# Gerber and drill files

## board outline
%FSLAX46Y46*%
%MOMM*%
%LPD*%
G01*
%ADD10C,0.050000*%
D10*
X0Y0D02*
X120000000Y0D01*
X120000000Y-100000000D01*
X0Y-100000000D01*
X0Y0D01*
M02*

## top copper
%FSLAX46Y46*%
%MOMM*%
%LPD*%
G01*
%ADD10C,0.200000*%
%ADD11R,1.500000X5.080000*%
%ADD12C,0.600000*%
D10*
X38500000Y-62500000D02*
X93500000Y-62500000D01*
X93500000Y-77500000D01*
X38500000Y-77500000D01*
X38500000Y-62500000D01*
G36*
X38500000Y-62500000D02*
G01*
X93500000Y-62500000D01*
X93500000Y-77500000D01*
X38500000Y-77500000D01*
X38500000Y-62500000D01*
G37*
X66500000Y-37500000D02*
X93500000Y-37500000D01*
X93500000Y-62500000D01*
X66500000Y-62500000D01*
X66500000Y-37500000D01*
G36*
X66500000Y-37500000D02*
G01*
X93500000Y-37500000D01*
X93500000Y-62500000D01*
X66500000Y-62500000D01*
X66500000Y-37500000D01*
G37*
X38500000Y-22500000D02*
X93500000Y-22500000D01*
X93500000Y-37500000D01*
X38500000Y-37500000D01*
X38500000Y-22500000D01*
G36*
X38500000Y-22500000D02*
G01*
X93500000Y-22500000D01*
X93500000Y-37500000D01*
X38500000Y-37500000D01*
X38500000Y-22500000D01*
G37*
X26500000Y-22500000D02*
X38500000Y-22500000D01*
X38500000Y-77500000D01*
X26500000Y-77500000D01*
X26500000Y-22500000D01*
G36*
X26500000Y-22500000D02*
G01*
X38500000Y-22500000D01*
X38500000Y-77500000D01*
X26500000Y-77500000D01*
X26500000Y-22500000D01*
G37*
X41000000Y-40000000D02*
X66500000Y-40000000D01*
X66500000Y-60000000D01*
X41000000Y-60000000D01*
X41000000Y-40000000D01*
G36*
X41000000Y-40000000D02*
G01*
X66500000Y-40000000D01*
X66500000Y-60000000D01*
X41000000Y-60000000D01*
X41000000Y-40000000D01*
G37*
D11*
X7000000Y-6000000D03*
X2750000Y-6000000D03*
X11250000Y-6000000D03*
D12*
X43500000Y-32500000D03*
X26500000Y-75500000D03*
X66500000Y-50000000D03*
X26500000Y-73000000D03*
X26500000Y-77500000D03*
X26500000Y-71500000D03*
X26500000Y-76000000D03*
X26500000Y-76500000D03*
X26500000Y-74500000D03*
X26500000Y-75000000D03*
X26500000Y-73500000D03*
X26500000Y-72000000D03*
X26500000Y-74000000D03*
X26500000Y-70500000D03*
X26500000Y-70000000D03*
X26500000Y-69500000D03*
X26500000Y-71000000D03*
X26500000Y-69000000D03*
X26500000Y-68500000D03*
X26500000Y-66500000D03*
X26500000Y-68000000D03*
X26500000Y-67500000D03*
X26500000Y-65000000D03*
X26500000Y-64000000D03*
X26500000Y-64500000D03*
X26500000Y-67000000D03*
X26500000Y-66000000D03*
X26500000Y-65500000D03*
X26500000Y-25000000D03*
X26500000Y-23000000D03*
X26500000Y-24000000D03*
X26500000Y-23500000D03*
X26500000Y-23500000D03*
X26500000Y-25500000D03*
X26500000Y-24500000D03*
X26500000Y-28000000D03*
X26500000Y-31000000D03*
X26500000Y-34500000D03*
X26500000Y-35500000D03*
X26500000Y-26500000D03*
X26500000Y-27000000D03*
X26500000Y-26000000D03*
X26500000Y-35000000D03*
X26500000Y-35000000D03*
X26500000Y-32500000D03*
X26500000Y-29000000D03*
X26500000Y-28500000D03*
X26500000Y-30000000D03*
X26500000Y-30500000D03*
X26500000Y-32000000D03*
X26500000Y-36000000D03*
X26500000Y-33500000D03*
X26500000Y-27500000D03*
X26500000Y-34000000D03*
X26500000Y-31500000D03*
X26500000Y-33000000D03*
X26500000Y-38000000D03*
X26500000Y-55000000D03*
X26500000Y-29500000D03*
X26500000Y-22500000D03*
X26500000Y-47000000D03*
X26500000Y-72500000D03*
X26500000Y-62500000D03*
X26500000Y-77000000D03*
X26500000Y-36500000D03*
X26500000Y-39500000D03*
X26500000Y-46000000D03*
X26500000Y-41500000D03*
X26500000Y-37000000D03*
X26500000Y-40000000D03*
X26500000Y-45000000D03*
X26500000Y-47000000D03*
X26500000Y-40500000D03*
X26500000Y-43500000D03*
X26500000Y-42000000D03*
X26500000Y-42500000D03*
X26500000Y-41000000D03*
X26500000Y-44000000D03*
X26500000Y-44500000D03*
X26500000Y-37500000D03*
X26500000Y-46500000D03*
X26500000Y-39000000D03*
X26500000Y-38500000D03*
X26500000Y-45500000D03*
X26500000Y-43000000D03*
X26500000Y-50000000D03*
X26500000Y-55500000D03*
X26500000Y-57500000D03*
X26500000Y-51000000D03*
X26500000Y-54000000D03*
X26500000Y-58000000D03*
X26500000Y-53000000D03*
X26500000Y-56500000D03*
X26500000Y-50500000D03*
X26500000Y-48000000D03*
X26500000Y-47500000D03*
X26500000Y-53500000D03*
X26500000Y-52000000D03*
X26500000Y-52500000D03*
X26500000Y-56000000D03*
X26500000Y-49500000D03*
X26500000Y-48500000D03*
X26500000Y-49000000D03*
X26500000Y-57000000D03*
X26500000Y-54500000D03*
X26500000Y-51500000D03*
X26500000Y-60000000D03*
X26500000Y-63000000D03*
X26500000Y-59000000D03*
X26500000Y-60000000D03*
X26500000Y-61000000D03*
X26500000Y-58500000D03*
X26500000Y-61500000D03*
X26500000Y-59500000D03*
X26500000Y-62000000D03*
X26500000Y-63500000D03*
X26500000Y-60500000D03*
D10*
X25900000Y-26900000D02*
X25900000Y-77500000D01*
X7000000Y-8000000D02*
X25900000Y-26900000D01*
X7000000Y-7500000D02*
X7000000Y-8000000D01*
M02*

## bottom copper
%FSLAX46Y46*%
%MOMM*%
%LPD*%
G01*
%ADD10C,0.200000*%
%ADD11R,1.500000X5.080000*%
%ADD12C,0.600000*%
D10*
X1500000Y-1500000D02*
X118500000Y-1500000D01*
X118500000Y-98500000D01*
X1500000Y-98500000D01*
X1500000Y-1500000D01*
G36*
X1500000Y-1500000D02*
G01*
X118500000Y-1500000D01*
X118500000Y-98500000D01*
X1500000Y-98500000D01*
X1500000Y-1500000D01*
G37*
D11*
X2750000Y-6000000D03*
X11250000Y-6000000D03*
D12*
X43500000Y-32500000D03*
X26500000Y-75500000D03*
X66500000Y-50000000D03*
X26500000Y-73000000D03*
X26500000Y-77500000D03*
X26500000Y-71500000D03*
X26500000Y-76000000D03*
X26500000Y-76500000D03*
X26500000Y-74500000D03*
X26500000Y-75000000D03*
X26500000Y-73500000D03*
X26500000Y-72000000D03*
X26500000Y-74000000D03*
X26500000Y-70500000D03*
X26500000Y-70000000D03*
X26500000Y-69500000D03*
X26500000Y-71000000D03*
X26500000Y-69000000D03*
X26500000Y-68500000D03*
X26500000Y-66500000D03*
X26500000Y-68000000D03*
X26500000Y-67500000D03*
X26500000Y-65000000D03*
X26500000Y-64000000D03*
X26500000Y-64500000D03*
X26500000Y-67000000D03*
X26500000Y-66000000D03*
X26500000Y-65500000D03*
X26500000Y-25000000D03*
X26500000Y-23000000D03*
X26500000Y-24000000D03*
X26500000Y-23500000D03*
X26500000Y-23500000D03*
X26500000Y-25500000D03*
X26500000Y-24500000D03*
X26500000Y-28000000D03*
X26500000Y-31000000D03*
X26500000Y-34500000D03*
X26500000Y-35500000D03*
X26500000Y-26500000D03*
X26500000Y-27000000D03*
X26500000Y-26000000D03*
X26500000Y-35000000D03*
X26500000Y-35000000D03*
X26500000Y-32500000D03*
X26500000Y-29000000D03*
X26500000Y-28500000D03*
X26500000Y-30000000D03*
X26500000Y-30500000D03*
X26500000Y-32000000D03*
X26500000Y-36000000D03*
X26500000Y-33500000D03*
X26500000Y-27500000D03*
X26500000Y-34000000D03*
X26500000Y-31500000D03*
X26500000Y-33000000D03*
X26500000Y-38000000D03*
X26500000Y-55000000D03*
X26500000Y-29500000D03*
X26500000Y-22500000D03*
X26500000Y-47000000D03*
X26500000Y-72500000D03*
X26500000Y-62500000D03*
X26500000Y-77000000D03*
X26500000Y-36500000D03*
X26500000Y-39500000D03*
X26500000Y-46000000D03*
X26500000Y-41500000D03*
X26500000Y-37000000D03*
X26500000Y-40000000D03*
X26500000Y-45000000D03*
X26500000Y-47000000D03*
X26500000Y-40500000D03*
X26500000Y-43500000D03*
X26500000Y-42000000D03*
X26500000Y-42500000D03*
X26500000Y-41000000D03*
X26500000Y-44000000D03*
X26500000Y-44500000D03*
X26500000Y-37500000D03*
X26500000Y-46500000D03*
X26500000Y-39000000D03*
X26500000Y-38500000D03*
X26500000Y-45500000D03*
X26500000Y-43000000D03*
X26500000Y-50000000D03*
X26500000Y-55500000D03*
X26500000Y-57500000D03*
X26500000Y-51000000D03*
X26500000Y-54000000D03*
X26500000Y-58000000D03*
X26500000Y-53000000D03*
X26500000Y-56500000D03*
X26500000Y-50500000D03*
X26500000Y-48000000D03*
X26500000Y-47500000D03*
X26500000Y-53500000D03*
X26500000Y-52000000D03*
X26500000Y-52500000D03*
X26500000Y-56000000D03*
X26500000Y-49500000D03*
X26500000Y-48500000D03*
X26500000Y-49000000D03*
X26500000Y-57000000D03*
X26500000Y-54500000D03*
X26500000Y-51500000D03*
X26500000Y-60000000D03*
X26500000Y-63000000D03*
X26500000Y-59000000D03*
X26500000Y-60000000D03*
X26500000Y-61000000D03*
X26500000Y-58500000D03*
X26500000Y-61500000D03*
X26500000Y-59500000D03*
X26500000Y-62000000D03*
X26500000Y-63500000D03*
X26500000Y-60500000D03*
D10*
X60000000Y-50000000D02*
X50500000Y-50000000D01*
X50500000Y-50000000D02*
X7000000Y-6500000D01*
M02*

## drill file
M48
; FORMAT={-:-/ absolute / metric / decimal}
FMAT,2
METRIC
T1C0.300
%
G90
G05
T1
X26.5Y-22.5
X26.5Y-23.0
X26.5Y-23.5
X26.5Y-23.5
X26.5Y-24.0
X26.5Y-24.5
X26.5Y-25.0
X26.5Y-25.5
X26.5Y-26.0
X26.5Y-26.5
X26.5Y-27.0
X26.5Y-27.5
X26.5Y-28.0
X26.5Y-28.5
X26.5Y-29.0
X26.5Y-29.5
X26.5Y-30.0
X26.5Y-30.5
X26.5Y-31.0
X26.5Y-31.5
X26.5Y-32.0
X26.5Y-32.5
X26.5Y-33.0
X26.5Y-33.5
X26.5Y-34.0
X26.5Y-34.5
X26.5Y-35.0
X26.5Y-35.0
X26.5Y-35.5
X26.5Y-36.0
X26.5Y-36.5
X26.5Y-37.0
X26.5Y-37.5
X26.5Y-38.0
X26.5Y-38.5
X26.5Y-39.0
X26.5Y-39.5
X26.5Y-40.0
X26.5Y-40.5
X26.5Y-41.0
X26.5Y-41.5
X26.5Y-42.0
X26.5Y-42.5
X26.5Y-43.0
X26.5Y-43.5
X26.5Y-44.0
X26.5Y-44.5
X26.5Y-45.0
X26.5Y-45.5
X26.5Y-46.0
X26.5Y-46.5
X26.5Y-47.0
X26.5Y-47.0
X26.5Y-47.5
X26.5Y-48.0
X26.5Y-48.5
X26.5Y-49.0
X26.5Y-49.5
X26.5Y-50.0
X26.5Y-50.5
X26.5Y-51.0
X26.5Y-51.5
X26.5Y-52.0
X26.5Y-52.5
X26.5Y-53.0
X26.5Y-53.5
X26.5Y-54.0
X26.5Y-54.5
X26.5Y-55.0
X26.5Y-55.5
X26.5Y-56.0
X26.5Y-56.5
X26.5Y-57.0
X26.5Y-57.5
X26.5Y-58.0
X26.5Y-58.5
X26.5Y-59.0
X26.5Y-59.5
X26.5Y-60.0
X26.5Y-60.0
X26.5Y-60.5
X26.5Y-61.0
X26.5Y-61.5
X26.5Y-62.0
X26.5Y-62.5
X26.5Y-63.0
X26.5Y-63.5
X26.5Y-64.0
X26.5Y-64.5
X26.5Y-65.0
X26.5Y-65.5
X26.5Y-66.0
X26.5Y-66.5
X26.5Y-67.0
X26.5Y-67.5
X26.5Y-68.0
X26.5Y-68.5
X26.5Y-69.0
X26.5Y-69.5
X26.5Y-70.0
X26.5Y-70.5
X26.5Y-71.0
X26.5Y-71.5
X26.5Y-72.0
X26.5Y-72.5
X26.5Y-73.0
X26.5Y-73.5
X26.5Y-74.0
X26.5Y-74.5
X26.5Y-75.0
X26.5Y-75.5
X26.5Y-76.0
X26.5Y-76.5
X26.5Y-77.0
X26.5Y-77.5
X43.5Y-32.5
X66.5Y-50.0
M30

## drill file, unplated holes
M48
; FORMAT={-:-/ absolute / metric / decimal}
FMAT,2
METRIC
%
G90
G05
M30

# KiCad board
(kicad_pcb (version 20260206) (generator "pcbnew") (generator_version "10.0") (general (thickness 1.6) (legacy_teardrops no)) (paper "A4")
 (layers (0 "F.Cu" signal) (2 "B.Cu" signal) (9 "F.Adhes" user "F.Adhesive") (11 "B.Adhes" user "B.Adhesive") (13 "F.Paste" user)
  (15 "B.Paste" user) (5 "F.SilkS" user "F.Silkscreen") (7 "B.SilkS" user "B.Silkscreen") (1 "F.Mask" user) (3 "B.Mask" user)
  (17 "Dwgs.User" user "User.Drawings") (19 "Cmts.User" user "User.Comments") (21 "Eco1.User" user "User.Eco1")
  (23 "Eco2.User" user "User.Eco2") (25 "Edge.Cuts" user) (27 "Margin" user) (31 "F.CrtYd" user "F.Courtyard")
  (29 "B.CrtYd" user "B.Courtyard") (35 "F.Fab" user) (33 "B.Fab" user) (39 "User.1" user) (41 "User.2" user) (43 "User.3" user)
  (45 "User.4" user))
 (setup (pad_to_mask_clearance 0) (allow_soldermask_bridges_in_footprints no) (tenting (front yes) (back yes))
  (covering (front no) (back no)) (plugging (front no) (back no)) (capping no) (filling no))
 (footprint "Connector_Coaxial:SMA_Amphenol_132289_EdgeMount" (layer "F.Cu") (at 7 6 90)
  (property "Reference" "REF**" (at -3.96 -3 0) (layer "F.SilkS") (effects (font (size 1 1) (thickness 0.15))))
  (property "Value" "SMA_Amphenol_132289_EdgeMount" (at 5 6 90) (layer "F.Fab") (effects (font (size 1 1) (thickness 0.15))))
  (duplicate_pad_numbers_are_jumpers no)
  (pad "1" smd rect (at 0 0 180) (size 1.5 5.08) (layers "F.Cu" "F.Mask" "F.Paste") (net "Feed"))
  (pad "2" smd rect (at 0 -4.25 180) (size 1.5 5.08) (layers "F.Cu" "F.Mask" "F.Paste"))
  (pad "2" smd rect (at 0 -4.25 180) (size 1.5 5.08) (layers "B.Cu" "B.Mask" "B.Paste") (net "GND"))
  (pad "2" smd rect (at 0 4.25 180) (size 1.5 5.08) (layers "F.Cu" "F.Mask" "F.Paste"))
  (pad "2" smd rect (at 0 4.25 180) (size 1.5 5.08) (layers "B.Cu" "B.Mask" "B.Paste") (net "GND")))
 (gr_rect (start 26.5 22.5) (end 38.5 77.5) (stroke (width 0.2) (type default)) (fill yes) (layer "F.Cu") (net "GND"))
 (gr_rect (start 38.5 22.5) (end 93.5 37.5) (stroke (width 0.2) (type default)) (fill yes) (layer "F.Cu") (net "GND"))
 (gr_rect (start 38.5 62.5) (end 93.5 77.5) (stroke (width 0.2) (type default)) (fill yes) (layer "F.Cu") (net "GND"))
 (gr_rect (start 41 40) (end 66.5 60) (stroke (width 0.2) (type default)) (fill yes) (layer "F.Cu") (net "GND"))
 (gr_rect (start 66.5 37.5) (end 93.5 62.5) (stroke (width 0.2) (type default)) (fill yes) (layer "F.Cu") (net "GND"))
 (gr_rect (start 1.5 1.5) (end 118.5 98.5) (stroke (width 0.2) (type solid)) (fill yes) (layer "B.Cu") (net "GND"))
 (gr_rect (start 0 0) (end 120 100) (stroke (width 0.05) (type default)) (fill no) (layer "Edge.Cuts"))
 (segment (start 7 8) (end 25.9 26.9) (width 0.2) (layer "F.Cu") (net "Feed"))
 (segment (start 7 7.5) (end 7 8) (width 0.2) (layer "F.Cu") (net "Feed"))
 (segment (start 25.9 26.9) (end 25.9 77.5) (width 0.2) (layer "F.Cu") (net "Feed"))
 (via (at 26.5 41.5) (size 0.6) (drill 0.3) (layers "F.Cu" "B.Cu") (free yes) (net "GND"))
 (via (at 26.5 47.5) (size 0.6) (drill 0.3) (layers "F.Cu" "B.Cu") (free yes) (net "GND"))
 (via (at 26.5 51.5) (size 0.6) (drill 0.3) (layers "F.Cu" "B.Cu") (free yes) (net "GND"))
 (via (at 26.5 53.5) (size 0.6) (drill 0.3) (layers "F.Cu" "B.Cu") (free yes) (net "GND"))
 (via (at 26.5 25) (size 0.6) (drill 0.3) (layers "F.Cu" "B.Cu") (free yes) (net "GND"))
 (via (at 26.5 30) (size 0.6) (drill 0.3) (layers "F.Cu" "B.Cu") (free yes) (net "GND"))
 (via (at 26.5 55.5) (size 0.6) (drill 0.3) (layers "F.Cu" "B.Cu") (free yes) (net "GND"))
 (via (at 26.5 29) (size 0.6) (drill 0.3) (layers "F.Cu" "B.Cu") (free yes) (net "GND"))
 (via (at 26.5 35) (size 0.6) (drill 0.3) (layers "F.Cu" "B.Cu") (free yes) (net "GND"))
 (via (at 26.5 55) (size 0.6) (drill 0.3) (layers "F.Cu" "B.Cu") (free yes) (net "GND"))
 (via (at 26.5 34.5) (size 0.6) (drill 0.3) (layers "F.Cu" "B.Cu") (free yes) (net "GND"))
 (via (at 26.5 24) (size 0.6) (drill 0.3) (layers "F.Cu" "B.Cu") (free yes) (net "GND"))
 (via (at 26.5 71.5) (size 0.6) (drill 0.3) (layers "F.Cu" "B.Cu") (free yes) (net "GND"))
 (via (at 26.5 68) (size 0.6) (drill 0.3) (layers "F.Cu" "B.Cu") (free yes) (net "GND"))
 (via (at 26.5 64.5) (size 0.6) (drill 0.3) (layers "F.Cu" "B.Cu") (free yes) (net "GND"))
 (via (at 26.5 26) (size 0.6) (drill 0.3) (layers "F.Cu" "B.Cu") (free yes) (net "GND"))
 (via (at 26.5 46.5) (size 0.6) (drill 0.3) (layers "F.Cu" "B.Cu") (free yes) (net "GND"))
 (via (at 26.5 53) (size 0.6) (drill 0.3) (layers "F.Cu" "B.Cu") (free yes) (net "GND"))
 (via (at 26.5 54) (size 0.6) (drill 0.3) (layers "F.Cu" "B.Cu") (free yes) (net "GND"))
 (via (at 26.5 62) (size 0.6) (drill 0.3) (layers "F.Cu" "B.Cu") (free yes) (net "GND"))
 (via (at 26.5 32) (size 0.6) (drill 0.3) (layers "F.Cu" "B.Cu") (free yes) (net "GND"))
 (via (at 26.5 50) (size 0.6) (drill 0.3) (layers "F.Cu" "B.Cu") (free yes) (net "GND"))
 (via (at 26.5 47) (size 0.6) (drill 0.3) (layers "F.Cu" "B.Cu") (free yes) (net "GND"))
 (via (at 26.5 29.5) (size 0.6) (drill 0.3) (layers "F.Cu" "B.Cu") (free yes) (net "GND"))
 (via (at 26.5 45.5) (size 0.6) (drill 0.3) (layers "F.Cu" "B.Cu") (free yes) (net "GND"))
 (via (at 26.5 52.5) (size 0.6) (drill 0.3) (layers "F.Cu" "B.Cu") (free yes) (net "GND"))
 (via (at 26.5 68.5) (size 0.6) (drill 0.3) (layers "F.Cu" "B.Cu") (free yes) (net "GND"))
 (via (at 26.5 57) (size 0.6) (drill 0.3) (layers "F.Cu" "B.Cu") (free yes) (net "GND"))
 (via (at 26.5 33) (size 0.6) (drill 0.3) (layers "F.Cu" "B.Cu") (free yes) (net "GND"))
 (via (at 26.5 36) (size 0.6) (drill 0.3) (layers "F.Cu" "B.Cu") (free yes) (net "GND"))
 (via (at 26.5 30.5) (size 0.6) (drill 0.3) (layers "F.Cu" "B.Cu") (free yes) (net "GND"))
 (via (at 26.5 66) (size 0.6) (drill 0.3) (layers "F.Cu" "B.Cu") (free yes) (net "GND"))
 (via (at 26.5 67) (size 0.6) (drill 0.3) (layers "F.Cu" "B.Cu") (free yes) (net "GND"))
 (via (at 26.5 63.5) (size 0.6) (drill 0.3) (layers "F.Cu" "B.Cu") (free yes) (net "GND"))
 (via (at 26.5 66.5) (size 0.6) (drill 0.3) (layers "F.Cu" "B.Cu") (free yes) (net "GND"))
 (via (at 26.5 56.5) (size 0.6) (drill 0.3) (layers "F.Cu" "B.Cu") (free yes) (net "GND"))
 (via (at 26.5 61.5) (size 0.6) (drill 0.3) (layers "F.Cu" "B.Cu") (free yes) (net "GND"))
 (via (at 26.5 43.5) (size 0.6) (drill 0.3) (layers "F.Cu" "B.Cu") (free yes) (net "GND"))
 (via (at 26.5 65) (size 0.6) (drill 0.3) (layers "F.Cu" "B.Cu") (free yes) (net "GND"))
 (via (at 26.5 32.5) (size 0.6) (drill 0.3) (layers "F.Cu" "B.Cu") (free yes) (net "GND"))
 (via (at 26.5 60.5) (size 0.6) (drill 0.3) (layers "F.Cu" "B.Cu") (free yes) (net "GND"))
 (via (at 26.5 26.5) (size 0.6) (drill 0.3) (layers "F.Cu" "B.Cu") (free yes) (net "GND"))
 (via (at 26.5 77.5) (size 0.6) (drill 0.3) (layers "F.Cu" "B.Cu") (free yes) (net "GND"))
 (via (at 26.5 72.5) (size 0.6) (drill 0.3) (layers "F.Cu" "B.Cu") (free yes) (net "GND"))
 (via (at 26.5 75.5) (size 0.6) (drill 0.3) (layers "F.Cu" "B.Cu") (free yes) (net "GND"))
 (via (at 26.5 56) (size 0.6) (drill 0.3) (layers "F.Cu" "B.Cu") (free yes) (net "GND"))
 (via (at 26.5 49.5) (size 0.6) (drill 0.3) (layers "F.Cu" "B.Cu") (free yes) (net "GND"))
 (via (at 26.5 70.5) (size 0.6) (drill 0.3) (layers "F.Cu" "B.Cu") (free yes) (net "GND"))
 (via (at 26.5 49) (size 0.6) (drill 0.3) (layers "F.Cu" "B.Cu") (free yes) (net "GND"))
 (via (at 26.5 23.5) (size 0.6) (drill 0.3) (layers "F.Cu" "B.Cu") (free yes) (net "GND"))
 (via (at 26.5 67.5) (size 0.6) (drill 0.3) (layers "F.Cu" "B.Cu") (free yes) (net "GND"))
 (via (at 26.5 44) (size 0.6) (drill 0.3) (layers "F.Cu" "B.Cu") (free yes) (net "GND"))
 (via (at 26.5 60) (size 0.6) (drill 0.3) (layers "F.Cu" "B.Cu") (free yes) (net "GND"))
 (via (at 26.5 27) (size 0.6) (drill 0.3) (layers "F.Cu" "B.Cu") (free yes) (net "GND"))
 (via (at 26.5 69.5) (size 0.6) (drill 0.3) (layers "F.Cu" "B.Cu") (free yes) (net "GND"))
 (via (at 26.5 71) (size 0.6) (drill 0.3) (layers "F.Cu" "B.Cu") (free yes) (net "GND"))
 (via (at 26.5 73) (size 0.6) (drill 0.3) (layers "F.Cu" "B.Cu") (free yes) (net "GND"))
 (via (at 26.5 48.5) (size 0.6) (drill 0.3) (layers "F.Cu" "B.Cu") (free yes) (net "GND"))
 (via (at 26.5 31.5) (size 0.6) (drill 0.3) (layers "F.Cu" "B.Cu") (free yes) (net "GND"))
 (via (at 26.5 52) (size 0.6) (drill 0.3) (layers "F.Cu" "B.Cu") (free yes) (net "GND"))
 (via (at 26.5 38) (size 0.6) (drill 0.3) (layers "F.Cu" "B.Cu") (free yes) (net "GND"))
 (via (at 26.5 34) (size 0.6) (drill 0.3) (layers "F.Cu" "B.Cu") (free yes) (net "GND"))
 (via (at 26.5 27.5) (size 0.6) (drill 0.3) (layers "F.Cu" "B.Cu") (free yes) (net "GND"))
 (via (at 26.5 38.5) (size 0.6) (drill 0.3) (layers "F.Cu" "B.Cu") (free yes) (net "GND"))
 (via (at 26.5 58) (size 0.6) (drill 0.3) (layers "F.Cu" "B.Cu") (free yes) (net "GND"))
 (via (at 26.5 63) (size 0.6) (drill 0.3) (layers "F.Cu" "B.Cu") (free yes) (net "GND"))
 (via (at 26.5 64) (size 0.6) (drill 0.3) (layers "F.Cu" "B.Cu") (free yes) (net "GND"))
 (via (at 66.5 50) (size 0.6) (drill 0.3) (layers "F.Cu" "B.Cu") (free yes) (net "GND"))
 (via (at 26.5 40) (size 0.6) (drill 0.3) (layers "F.Cu" "B.Cu") (free yes) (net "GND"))
 (via (at 26.5 62.5) (size 0.6) (drill 0.3) (layers "F.Cu" "B.Cu") (free yes) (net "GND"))
 (via (at 26.5 65.5) (size 0.6) (drill 0.3) (layers "F.Cu" "B.Cu") (free yes) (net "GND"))
 (via (at 26.5 69) (size 0.6) (drill 0.3) (layers "F.Cu" "B.Cu") (free yes) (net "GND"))
 (via (at 26.5 73.5) (size 0.6) (drill 0.3) (layers "F.Cu" "B.Cu") (free yes) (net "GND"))
 (via (at 26.5 22.5) (size 0.6) (drill 0.3) (layers "F.Cu" "B.Cu") (free yes) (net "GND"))
 (via (at 26.5 61) (size 0.6) (drill 0.3) (layers "F.Cu" "B.Cu") (free yes) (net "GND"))
 (via (at 26.5 59) (size 0.6) (drill 0.3) (layers "F.Cu" "B.Cu") (free yes) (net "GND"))
 (via (at 26.5 70) (size 0.6) (drill 0.3) (layers "F.Cu" "B.Cu") (free yes) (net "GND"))
 (via (at 26.5 42.5) (size 0.6) (drill 0.3) (layers "F.Cu" "B.Cu") (free yes) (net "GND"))
 (via (at 26.5 47) (size 0.6) (drill 0.3) (layers "F.Cu" "B.Cu") (free yes) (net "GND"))
 (via (at 26.5 43) (size 0.6) (drill 0.3) (layers "F.Cu" "B.Cu") (free yes) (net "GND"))
 (via (at 26.5 28.5) (size 0.6) (drill 0.3) (layers "F.Cu" "B.Cu") (free yes) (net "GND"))
 (via (at 26.5 37.5) (size 0.6) (drill 0.3) (layers "F.Cu" "B.Cu") (free yes) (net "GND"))
 (via (at 26.5 45) (size 0.6) (drill 0.3) (layers "F.Cu" "B.Cu") (free yes) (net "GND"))
 (via (at 26.5 60) (size 0.6) (drill 0.3) (layers "F.Cu" "B.Cu") (free yes) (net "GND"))
 (via (at 26.5 58.5) (size 0.6) (drill 0.3) (layers "F.Cu" "B.Cu") (free yes) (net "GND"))
 (via (at 43.5 32.5) (size 0.6) (drill 0.3) (layers "F.Cu" "B.Cu") (free yes) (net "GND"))
 (via (at 26.5 40.5) (size 0.6) (drill 0.3) (layers "F.Cu" "B.Cu") (free yes) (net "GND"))
 (via (at 26.5 23) (size 0.6) (drill 0.3) (layers "F.Cu" "B.Cu") (free yes) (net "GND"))
 (via (at 26.5 59.5) (size 0.6) (drill 0.3) (layers "F.Cu" "B.Cu") (free yes) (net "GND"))
 (via (at 26.5 72) (size 0.6) (drill 0.3) (layers "F.Cu" "B.Cu") (free yes) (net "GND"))
 (via (at 26.5 76) (size 0.6) (drill 0.3) (layers "F.Cu" "B.Cu") (free yes) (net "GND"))
 (via (at 26.5 74.5) (size 0.6) (drill 0.3) (layers "F.Cu" "B.Cu") (free yes) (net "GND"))
 (via (at 26.5 35.5) (size 0.6) (drill 0.3) (layers "F.Cu" "B.Cu") (free yes) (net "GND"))
 (via (at 26.5 39.5) (size 0.6) (drill 0.3) (layers "F.Cu" "B.Cu") (free yes) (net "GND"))
 (via (at 26.5 42) (size 0.6) (drill 0.3) (layers "F.Cu" "B.Cu") (free yes) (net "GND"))
 (via (at 26.5 36.5) (size 0.6) (drill 0.3) (layers "F.Cu" "B.Cu") (free yes) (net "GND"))
 (via (at 26.5 23.5) (size 0.6) (drill 0.3) (layers "F.Cu" "B.Cu") (free yes) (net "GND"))
 (via (at 26.5 39) (size 0.6) (drill 0.3) (layers "F.Cu" "B.Cu") (free yes) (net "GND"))
 (via (at 26.5 31) (size 0.6) (drill 0.3) (layers "F.Cu" "B.Cu") (free yes) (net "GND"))
 (via (at 26.5 48) (size 0.6) (drill 0.3) (layers "F.Cu" "B.Cu") (free yes) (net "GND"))
 (via (at 26.5 44.5) (size 0.6) (drill 0.3) (layers "F.Cu" "B.Cu") (free yes) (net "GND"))
 (via (at 26.5 54.5) (size 0.6) (drill 0.3) (layers "F.Cu" "B.Cu") (free yes) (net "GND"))
 (via (at 26.5 24.5) (size 0.6) (drill 0.3) (layers "F.Cu" "B.Cu") (free yes) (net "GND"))
 (via (at 26.5 75) (size 0.6) (drill 0.3) (layers "F.Cu" "B.Cu") (free yes) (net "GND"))
 (via (at 26.5 25.5) (size 0.6) (drill 0.3) (layers "F.Cu" "B.Cu") (free yes) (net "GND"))
 (via (at 26.5 37) (size 0.6) (drill 0.3) (layers "F.Cu" "B.Cu") (free yes) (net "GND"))
 (via (at 26.5 50.5) (size 0.6) (drill 0.3) (layers "F.Cu" "B.Cu") (free yes) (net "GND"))
 (via (at 26.5 74) (size 0.6) (drill 0.3) (layers "F.Cu" "B.Cu") (free yes) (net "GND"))
 (via (at 26.5 51) (size 0.6) (drill 0.3) (layers "F.Cu" "B.Cu") (free yes) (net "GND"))
 (via (at 26.5 35) (size 0.6) (drill 0.3) (layers "F.Cu" "B.Cu") (free yes) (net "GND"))
 (via (at 26.5 76.5) (size 0.6) (drill 0.3) (layers "F.Cu" "B.Cu") (free yes) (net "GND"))
 (via (at 26.5 77) (size 0.6) (drill 0.3) (layers "F.Cu" "B.Cu") (free yes) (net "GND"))
 (via (at 26.5 33.5) (size 0.6) (drill 0.3) (layers "F.Cu" "B.Cu") (free yes) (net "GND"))
 (via (at 26.5 46) (size 0.6) (drill 0.3) (layers "F.Cu" "B.Cu") (free yes) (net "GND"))
 (via (at 26.5 41) (size 0.6) (drill 0.3) (layers "F.Cu" "B.Cu") (free yes) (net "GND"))
 (via (at 26.5 28) (size 0.6) (drill 0.3) (layers "F.Cu" "B.Cu") (free yes) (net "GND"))
 (via (at 26.5 57.5) (size 0.6) (drill 0.3) (layers "F.Cu" "B.Cu") (free yes) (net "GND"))
 (segment (start 50.5 50) (end 7 6.5) (width 0.2) (layer "B.Cu") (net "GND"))
 (segment (start 60 50) (end 50.5 50) (width 0.2) (layer "B.Cu") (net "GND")))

